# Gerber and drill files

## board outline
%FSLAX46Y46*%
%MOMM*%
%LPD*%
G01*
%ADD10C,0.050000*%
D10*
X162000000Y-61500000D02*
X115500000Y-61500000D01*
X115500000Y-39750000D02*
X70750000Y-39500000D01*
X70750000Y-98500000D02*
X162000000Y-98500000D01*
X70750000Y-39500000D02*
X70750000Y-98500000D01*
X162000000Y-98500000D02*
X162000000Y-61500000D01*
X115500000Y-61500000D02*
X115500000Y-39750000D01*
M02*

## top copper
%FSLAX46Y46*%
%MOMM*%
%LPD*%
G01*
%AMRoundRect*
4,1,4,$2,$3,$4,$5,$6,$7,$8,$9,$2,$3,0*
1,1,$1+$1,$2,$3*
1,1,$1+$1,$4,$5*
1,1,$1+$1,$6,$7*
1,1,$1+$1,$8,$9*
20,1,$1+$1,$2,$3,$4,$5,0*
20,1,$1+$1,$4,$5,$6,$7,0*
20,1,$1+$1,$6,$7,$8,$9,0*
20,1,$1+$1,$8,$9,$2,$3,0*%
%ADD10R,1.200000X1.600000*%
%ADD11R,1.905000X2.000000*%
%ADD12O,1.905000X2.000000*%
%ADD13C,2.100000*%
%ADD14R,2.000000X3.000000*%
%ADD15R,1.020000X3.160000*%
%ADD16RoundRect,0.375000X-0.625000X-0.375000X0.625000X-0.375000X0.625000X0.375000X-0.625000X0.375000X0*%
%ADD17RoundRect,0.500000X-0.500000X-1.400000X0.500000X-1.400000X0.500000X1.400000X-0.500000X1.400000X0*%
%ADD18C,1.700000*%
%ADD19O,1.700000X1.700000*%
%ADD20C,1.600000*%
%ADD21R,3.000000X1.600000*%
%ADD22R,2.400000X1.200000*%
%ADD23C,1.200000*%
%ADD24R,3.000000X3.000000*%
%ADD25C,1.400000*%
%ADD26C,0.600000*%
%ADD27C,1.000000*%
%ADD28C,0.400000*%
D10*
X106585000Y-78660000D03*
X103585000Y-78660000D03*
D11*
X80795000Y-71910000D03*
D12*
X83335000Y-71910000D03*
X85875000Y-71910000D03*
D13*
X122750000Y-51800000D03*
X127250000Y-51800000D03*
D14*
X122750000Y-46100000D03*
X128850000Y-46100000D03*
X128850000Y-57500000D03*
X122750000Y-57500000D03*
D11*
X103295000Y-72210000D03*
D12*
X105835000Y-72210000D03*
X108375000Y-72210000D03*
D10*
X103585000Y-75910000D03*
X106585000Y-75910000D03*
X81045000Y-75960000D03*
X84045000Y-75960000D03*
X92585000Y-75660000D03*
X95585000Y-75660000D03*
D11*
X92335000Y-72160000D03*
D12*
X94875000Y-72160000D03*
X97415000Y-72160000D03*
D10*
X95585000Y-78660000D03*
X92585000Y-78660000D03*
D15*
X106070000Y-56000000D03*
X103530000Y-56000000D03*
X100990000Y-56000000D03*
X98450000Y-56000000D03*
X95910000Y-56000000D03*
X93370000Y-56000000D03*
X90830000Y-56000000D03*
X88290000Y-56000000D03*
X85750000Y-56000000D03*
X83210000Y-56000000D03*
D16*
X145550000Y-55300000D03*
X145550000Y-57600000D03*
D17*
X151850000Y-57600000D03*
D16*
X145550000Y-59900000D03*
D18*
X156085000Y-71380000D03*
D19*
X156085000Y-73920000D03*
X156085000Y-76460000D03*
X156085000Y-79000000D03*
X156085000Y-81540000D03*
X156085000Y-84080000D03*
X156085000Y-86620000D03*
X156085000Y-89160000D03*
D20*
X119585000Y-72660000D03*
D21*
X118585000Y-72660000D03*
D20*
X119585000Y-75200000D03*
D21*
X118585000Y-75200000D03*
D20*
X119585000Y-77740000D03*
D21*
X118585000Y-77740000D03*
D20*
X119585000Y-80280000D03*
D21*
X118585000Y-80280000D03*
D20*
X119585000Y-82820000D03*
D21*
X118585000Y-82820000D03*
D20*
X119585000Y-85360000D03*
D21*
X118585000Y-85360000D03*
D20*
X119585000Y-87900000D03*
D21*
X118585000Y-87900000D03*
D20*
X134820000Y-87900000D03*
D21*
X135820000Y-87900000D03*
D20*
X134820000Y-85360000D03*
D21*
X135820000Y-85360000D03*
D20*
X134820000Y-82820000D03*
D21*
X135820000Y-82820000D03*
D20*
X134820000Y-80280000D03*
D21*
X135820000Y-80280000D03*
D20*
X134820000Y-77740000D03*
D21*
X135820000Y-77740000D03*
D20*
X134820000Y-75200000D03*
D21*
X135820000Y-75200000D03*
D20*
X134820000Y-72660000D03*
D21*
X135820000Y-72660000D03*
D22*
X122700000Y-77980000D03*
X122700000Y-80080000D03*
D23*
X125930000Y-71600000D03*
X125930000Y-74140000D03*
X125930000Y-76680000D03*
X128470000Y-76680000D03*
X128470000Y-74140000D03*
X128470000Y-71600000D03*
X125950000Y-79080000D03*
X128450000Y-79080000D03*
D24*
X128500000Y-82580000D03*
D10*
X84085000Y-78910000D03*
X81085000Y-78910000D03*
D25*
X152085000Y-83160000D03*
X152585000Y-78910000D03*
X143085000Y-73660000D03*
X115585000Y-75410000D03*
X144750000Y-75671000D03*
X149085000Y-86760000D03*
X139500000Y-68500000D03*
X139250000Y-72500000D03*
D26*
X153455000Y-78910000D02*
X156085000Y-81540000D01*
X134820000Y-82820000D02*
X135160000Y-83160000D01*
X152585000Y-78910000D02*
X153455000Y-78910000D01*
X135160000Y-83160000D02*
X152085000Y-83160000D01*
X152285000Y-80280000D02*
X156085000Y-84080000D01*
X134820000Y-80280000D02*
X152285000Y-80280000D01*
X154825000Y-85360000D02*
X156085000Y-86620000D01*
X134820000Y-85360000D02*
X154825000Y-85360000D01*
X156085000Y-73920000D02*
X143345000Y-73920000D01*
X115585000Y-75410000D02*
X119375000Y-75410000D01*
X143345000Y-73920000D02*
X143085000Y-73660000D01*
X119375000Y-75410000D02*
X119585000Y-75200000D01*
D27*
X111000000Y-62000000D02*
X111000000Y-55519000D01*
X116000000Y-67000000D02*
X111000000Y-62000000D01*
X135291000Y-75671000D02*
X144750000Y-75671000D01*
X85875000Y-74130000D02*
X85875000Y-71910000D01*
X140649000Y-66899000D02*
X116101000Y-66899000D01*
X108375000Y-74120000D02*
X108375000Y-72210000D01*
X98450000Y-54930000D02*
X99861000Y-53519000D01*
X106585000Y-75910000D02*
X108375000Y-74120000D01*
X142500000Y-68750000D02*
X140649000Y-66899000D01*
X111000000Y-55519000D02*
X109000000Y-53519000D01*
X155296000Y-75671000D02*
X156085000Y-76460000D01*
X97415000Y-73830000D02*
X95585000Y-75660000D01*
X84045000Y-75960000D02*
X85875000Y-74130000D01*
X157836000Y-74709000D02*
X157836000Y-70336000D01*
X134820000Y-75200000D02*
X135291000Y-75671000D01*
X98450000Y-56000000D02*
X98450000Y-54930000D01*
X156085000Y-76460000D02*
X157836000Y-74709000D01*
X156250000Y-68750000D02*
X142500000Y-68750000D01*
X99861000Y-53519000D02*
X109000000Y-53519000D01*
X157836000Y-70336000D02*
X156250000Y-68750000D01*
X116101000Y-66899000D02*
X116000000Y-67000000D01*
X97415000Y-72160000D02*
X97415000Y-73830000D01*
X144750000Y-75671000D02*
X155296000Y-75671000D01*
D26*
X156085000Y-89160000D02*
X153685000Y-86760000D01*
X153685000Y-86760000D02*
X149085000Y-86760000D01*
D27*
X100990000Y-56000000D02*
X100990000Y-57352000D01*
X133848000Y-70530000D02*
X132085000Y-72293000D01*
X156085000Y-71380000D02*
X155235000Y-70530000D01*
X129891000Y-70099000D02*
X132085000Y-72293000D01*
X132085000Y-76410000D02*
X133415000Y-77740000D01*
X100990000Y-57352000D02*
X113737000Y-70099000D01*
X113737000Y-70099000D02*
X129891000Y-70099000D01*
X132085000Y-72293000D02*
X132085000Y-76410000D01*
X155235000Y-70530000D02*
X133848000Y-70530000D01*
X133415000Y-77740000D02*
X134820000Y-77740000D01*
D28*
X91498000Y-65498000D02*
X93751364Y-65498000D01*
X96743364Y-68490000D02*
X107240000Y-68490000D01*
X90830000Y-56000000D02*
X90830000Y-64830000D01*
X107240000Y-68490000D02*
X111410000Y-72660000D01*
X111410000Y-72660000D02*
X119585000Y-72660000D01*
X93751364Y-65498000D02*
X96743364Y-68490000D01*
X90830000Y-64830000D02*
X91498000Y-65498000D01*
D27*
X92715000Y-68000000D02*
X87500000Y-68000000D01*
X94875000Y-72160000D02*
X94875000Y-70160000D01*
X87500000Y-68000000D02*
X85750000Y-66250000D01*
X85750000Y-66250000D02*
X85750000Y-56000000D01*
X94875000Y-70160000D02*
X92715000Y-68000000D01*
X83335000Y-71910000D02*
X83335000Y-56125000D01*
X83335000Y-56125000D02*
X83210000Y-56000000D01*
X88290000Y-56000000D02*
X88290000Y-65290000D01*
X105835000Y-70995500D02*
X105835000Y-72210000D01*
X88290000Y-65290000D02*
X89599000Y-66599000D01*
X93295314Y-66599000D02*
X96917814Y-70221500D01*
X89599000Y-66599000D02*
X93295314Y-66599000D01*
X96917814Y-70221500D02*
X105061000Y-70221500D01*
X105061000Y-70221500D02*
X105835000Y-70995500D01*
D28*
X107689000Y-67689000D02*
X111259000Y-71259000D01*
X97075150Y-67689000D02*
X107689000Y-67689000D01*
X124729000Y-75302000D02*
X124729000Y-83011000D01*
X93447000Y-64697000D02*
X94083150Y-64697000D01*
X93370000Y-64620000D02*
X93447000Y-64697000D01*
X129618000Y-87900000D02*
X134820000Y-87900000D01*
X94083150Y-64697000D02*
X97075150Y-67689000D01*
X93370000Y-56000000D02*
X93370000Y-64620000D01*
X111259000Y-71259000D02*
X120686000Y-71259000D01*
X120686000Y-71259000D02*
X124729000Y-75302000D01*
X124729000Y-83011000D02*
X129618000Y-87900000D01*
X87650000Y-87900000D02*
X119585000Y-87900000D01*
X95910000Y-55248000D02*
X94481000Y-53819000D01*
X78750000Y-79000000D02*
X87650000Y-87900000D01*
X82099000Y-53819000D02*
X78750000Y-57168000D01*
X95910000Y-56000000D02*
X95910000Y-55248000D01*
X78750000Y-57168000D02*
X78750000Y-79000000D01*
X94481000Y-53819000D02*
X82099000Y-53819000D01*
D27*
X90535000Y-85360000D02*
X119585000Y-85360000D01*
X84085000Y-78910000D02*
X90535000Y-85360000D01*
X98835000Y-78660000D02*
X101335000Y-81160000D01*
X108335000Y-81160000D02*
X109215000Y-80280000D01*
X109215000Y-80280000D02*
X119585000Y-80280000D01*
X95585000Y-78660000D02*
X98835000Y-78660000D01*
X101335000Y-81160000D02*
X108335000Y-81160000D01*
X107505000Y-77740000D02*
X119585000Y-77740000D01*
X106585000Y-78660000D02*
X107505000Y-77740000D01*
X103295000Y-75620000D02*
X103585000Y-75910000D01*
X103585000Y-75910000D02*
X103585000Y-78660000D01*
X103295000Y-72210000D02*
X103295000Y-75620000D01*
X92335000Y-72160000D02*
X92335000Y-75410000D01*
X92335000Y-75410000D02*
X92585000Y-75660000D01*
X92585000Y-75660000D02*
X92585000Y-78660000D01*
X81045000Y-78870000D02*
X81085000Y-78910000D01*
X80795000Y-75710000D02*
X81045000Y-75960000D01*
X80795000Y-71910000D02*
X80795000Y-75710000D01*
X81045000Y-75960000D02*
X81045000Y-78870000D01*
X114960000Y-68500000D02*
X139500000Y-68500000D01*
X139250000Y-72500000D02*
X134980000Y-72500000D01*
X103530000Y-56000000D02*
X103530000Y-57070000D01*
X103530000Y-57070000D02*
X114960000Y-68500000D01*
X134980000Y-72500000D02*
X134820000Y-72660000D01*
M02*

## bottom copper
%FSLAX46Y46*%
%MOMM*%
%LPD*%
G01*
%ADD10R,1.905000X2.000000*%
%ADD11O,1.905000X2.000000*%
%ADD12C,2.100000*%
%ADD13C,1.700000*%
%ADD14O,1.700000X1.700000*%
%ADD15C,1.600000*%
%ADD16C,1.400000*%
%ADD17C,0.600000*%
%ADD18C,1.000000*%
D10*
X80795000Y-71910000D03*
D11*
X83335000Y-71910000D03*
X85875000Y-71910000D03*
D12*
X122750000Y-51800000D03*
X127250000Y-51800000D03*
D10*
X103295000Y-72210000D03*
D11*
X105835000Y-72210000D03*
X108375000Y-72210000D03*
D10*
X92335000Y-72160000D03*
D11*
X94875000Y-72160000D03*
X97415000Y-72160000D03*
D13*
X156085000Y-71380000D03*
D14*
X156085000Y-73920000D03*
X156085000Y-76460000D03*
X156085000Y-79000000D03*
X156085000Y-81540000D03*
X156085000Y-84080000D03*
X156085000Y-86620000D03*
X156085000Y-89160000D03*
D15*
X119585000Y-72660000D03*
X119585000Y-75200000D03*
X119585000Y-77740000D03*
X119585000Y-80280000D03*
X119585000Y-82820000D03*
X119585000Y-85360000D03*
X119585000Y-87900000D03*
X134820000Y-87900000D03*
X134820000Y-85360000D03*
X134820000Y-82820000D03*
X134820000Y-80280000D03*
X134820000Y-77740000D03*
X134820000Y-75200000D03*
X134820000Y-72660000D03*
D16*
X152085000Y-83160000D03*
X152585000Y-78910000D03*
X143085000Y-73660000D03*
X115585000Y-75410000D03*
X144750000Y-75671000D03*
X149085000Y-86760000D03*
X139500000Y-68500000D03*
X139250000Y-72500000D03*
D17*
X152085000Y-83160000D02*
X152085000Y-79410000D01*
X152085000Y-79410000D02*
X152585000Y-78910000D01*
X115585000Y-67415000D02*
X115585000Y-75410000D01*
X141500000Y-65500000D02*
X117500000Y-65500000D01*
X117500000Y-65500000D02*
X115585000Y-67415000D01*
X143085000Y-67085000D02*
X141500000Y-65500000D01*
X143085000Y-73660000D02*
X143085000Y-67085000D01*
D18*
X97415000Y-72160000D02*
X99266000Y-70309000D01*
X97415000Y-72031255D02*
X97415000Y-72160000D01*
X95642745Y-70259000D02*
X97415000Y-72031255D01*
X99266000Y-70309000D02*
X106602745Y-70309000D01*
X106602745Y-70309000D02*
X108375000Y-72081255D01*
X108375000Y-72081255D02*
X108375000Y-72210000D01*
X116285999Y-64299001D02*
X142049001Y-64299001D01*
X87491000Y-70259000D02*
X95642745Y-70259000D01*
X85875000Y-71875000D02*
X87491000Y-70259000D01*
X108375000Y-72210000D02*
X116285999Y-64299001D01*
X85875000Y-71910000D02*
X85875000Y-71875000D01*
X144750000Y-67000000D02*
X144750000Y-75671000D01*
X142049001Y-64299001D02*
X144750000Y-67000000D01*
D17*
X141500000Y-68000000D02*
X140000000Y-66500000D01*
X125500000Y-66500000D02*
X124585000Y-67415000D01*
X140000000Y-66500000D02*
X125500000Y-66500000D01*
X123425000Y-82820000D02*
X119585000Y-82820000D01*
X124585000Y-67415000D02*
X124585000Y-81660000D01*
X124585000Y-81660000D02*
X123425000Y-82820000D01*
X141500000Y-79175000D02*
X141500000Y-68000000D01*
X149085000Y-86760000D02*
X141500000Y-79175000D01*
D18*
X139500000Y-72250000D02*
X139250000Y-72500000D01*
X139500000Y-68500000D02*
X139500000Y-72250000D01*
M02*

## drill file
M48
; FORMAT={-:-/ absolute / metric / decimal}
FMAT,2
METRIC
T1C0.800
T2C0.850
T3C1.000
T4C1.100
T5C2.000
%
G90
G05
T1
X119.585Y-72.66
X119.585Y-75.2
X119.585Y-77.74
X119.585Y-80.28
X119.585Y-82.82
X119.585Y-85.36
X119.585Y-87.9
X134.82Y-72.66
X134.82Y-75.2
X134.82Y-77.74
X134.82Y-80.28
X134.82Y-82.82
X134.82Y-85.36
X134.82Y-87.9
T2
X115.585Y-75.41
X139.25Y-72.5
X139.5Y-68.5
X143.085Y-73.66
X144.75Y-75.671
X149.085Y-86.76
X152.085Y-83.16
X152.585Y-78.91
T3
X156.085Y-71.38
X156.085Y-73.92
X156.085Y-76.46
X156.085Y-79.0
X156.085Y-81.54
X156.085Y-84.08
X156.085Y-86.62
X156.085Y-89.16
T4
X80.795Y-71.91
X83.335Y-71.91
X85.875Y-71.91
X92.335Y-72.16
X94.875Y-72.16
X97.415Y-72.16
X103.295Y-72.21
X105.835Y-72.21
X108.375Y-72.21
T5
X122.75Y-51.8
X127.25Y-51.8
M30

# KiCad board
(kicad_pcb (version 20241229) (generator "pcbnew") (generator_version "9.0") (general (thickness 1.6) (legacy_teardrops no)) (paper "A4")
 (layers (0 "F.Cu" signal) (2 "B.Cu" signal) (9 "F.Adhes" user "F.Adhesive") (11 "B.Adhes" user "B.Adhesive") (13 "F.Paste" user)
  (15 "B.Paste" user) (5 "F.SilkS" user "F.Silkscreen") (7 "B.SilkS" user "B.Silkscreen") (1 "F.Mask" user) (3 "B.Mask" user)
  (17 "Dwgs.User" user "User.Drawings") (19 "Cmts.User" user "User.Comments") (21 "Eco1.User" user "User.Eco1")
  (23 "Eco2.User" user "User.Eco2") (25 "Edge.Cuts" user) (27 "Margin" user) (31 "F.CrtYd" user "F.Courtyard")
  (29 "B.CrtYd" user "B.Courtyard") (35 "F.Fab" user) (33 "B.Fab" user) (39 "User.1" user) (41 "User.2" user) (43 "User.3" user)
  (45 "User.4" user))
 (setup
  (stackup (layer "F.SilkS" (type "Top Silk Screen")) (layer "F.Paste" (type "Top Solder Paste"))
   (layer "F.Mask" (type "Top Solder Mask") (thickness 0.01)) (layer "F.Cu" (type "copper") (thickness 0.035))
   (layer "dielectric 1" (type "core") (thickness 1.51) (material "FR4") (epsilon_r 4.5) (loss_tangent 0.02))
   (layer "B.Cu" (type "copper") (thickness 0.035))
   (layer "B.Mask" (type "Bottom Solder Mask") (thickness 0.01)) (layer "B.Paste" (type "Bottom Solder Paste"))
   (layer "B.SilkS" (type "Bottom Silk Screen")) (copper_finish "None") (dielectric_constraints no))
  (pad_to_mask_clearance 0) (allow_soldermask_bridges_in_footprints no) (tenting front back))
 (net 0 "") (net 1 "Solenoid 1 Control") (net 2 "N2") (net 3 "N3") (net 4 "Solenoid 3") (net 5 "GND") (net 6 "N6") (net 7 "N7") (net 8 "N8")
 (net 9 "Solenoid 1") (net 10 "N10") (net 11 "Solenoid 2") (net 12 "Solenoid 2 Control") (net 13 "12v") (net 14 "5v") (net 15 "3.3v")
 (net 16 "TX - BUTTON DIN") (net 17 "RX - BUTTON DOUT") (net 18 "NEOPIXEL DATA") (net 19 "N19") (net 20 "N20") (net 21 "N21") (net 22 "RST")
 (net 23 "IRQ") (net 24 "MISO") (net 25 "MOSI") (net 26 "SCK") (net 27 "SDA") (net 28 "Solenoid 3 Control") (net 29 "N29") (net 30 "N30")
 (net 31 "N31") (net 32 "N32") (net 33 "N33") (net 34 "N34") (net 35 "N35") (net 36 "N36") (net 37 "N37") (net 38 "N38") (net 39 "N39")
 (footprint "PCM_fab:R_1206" (layer "F.Cu") (at 105.085 78.66 180)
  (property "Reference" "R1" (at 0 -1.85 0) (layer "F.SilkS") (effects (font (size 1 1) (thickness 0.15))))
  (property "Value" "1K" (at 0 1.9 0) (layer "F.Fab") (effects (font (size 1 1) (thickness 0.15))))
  (pad "1" smd rect (at -1.5 0 180) (size 1.2 1.6) (layers "F.Cu" "F.Mask" "F.Paste") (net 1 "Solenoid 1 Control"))
  (pad "2" smd rect (at 1.5 0 180) (size 1.2 1.6) (layers "F.Cu" "F.Mask" "F.Paste") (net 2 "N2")))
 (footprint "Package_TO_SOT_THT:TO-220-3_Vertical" (layer "F.Cu") (at 80.795 71.91)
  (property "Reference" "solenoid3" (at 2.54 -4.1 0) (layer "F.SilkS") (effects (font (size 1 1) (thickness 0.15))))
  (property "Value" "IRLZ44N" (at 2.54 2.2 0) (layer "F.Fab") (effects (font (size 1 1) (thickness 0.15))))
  (pad "1" thru_hole rect (at 0 0) (size 1.905 2) (drill 1.1) (layers "*.Cu" "*.Mask") (remove_unused_layers no) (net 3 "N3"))
  (pad "2" thru_hole oval (at 2.54 0) (size 1.905 2) (drill 1.1) (layers "*.Cu" "*.Mask") (remove_unused_layers no) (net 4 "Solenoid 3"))
  (pad "3" thru_hole oval (at 5.08 0) (size 1.905 2) (drill 1.1) (layers "*.Cu" "*.Mask") (remove_unused_layers no) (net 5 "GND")))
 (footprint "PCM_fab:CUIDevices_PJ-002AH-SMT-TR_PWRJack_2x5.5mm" (layer "F.Cu") (at 125.75 51.8)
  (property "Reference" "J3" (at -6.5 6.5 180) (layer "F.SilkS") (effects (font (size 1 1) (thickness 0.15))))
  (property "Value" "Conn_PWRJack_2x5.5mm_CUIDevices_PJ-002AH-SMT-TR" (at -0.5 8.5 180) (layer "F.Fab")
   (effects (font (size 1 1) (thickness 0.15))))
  (pad "" thru_hole circle (at -3 0 90) (size 2.1 2.1) (drill 2) (layers "*.Cu" "*.Mask") (remove_unused_layers no))
  (pad "" thru_hole circle (at 1.5 0 90) (size 2.1 2.1) (drill 2) (layers "*.Cu" "*.Mask") (remove_unused_layers no))
  (pad "1" smd rect (at -3 -5.7 90) (size 3 2) (layers "F.Cu" "F.Mask" "F.Paste") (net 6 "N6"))
  (pad "1" smd rect (at 3.1 -5.7 90) (size 3 2) (layers "F.Cu" "F.Mask" "F.Paste") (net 6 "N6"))
  (pad "2" smd rect (at 3.1 5.7 90) (size 3 2) (layers "F.Cu" "F.Mask" "F.Paste") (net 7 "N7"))
  (pad "3" smd rect (at -3 5.7 90) (size 3 2) (layers "F.Cu" "F.Mask" "F.Paste") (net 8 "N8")))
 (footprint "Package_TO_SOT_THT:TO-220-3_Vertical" (layer "F.Cu") (at 103.295 72.21)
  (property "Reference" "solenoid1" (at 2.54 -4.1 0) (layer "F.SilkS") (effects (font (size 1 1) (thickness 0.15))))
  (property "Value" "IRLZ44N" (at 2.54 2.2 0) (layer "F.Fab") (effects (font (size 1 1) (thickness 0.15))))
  (pad "1" thru_hole rect (at 0 0) (size 1.905 2) (drill 1.1) (layers "*.Cu" "*.Mask") (remove_unused_layers no) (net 2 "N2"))
  (pad "2" thru_hole oval (at 2.54 0) (size 1.905 2) (drill 1.1) (layers "*.Cu" "*.Mask") (remove_unused_layers no) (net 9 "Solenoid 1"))
  (pad "3" thru_hole oval (at 5.08 0) (size 1.905 2) (drill 1.1) (layers "*.Cu" "*.Mask") (remove_unused_layers no) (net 5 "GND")))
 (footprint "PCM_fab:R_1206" (layer "F.Cu") (at 105.085 75.91)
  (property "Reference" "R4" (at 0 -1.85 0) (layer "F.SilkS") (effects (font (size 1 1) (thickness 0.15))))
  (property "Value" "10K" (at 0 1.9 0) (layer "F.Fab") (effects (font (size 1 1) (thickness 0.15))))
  (pad "1" smd rect (at -1.5 0) (size 1.2 1.6) (layers "F.Cu" "F.Mask" "F.Paste") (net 2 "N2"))
  (pad "2" smd rect (at 1.5 0) (size 1.2 1.6) (layers "F.Cu" "F.Mask" "F.Paste") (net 5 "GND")))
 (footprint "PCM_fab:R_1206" (layer "F.Cu") (at 82.545 75.96)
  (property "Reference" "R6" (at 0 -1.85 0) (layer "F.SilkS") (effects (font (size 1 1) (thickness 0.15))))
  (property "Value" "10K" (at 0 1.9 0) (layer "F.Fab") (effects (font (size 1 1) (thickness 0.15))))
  (pad "1" smd rect (at -1.5 0) (size 1.2 1.6) (layers "F.Cu" "F.Mask" "F.Paste") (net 3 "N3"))
  (pad "2" smd rect (at 1.5 0) (size 1.2 1.6) (layers "F.Cu" "F.Mask" "F.Paste") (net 5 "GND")))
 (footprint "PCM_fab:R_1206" (layer "F.Cu") (at 94.085 75.66)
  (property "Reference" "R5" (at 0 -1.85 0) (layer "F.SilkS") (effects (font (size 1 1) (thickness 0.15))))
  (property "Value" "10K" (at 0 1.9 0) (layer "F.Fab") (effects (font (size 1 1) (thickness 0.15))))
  (pad "1" smd rect (at -1.5 0) (size 1.2 1.6) (layers "F.Cu" "F.Mask" "F.Paste") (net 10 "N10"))
  (pad "2" smd rect (at 1.5 0) (size 1.2 1.6) (layers "F.Cu" "F.Mask" "F.Paste") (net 5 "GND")))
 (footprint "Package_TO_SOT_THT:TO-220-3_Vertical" (layer "F.Cu") (at 92.335 72.16)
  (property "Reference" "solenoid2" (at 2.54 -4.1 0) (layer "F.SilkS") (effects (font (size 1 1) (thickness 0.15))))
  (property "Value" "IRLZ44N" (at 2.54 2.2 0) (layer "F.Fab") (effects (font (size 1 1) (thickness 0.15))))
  (pad "1" thru_hole rect (at 0 0) (size 1.905 2) (drill 1.1) (layers "*.Cu" "*.Mask") (remove_unused_layers no) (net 10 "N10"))
  (pad "2" thru_hole oval (at 2.54 0) (size 1.905 2) (drill 1.1) (layers "*.Cu" "*.Mask") (remove_unused_layers no) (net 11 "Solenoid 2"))
  (pad "3" thru_hole oval (at 5.08 0) (size 1.905 2) (drill 1.1) (layers "*.Cu" "*.Mask") (remove_unused_layers no) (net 5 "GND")))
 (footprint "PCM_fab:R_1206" (layer "F.Cu") (at 94.085 78.66 180)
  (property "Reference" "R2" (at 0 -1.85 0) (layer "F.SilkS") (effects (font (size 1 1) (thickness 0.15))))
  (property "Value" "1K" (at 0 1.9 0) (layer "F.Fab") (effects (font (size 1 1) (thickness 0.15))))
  (pad "1" smd rect (at -1.5 0 180) (size 1.2 1.6) (layers "F.Cu" "F.Mask" "F.Paste") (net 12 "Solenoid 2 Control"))
  (pad "2" smd rect (at 1.5 0 180) (size 1.2 1.6) (layers "F.Cu" "F.Mask" "F.Paste") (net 10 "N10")))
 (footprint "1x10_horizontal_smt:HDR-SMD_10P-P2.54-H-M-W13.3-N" (layer "F.Cu") (at 94.64 56 180)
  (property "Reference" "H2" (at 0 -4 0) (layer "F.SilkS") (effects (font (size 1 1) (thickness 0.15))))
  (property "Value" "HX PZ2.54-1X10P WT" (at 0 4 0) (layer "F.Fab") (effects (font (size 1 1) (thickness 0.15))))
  (pad "1" smd rect (at -11.43 0 180) (size 1.02 3.16) (layers "F.Cu" "F.Mask" "F.Paste") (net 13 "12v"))
  (pad "2" smd rect (at -8.89 0 180) (size 1.02 3.16) (layers "F.Cu" "F.Mask" "F.Paste") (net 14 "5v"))
  (pad "3" smd rect (at -6.35 0 180) (size 1.02 3.16) (layers "F.Cu" "F.Mask" "F.Paste") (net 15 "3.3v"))
  (pad "4" smd rect (at -3.81 0 180) (size 1.02 3.16) (layers "F.Cu" "F.Mask" "F.Paste") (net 5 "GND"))
  (pad "5" smd rect (at -1.27 0 180) (size 1.02 3.16) (layers "F.Cu" "F.Mask" "F.Paste") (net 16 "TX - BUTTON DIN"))
  (pad "6" smd rect (at 1.27 0 180) (size 1.02 3.16) (layers "F.Cu" "F.Mask" "F.Paste") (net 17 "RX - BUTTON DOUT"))
  (pad "7" smd rect (at 3.81 0 180) (size 1.02 3.16) (layers "F.Cu" "F.Mask" "F.Paste") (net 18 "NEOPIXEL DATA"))
  (pad "8" smd rect (at 6.35 0 180) (size 1.02 3.16) (layers "F.Cu" "F.Mask" "F.Paste") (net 9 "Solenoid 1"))
  (pad "9" smd rect (at 8.89 0 180) (size 1.02 3.16) (layers "F.Cu" "F.Mask" "F.Paste") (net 11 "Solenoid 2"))
  (pad "10" smd rect (at 11.43 0 180) (size 1.02 3.16) (layers "F.Cu" "F.Mask" "F.Paste") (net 4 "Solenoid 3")))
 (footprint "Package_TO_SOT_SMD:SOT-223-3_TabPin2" (layer "F.Cu") (at 148.7 57.6)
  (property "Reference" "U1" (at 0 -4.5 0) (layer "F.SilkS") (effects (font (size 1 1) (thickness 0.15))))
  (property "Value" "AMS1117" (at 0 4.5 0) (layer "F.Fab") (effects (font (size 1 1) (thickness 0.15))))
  (pad "1" smd roundrect (at -3.15 -2.3) (size 2 1.5) (layers "F.Cu" "F.Mask" "F.Paste") (roundrect_rratio 0.25) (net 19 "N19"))
  (pad "2" smd roundrect (at -3.15 0) (size 2 1.5) (layers "F.Cu" "F.Mask" "F.Paste") (roundrect_rratio 0.25) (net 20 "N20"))
  (pad "2" smd roundrect (at 3.15 0) (size 2 3.8) (layers "F.Cu" "F.Mask" "F.Paste") (roundrect_rratio 0.25) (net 20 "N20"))
  (pad "3" smd roundrect (at -3.15 2.3) (size 2 1.5) (layers "F.Cu" "F.Mask" "F.Paste") (roundrect_rratio 0.25) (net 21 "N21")))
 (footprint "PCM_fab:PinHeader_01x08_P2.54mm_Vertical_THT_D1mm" (layer "F.Cu") (at 156.085 71.38)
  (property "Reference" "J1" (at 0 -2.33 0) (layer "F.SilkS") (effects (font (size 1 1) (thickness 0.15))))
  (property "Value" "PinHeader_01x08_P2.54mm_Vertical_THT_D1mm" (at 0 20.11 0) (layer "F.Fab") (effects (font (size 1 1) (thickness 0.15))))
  (pad "1" thru_hole circle (at 0 0) (size 1.7 1.7) (drill 1) (layers "*.Cu" "*.Mask") (remove_unused_layers no) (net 15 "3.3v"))
  (pad "2" thru_hole oval (at 0 2.54) (size 1.7 1.7) (drill 1) (layers "*.Cu" "*.Mask") (remove_unused_layers no) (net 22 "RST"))
  (pad "3" thru_hole oval (at 0 5.08) (size 1.7 1.7) (drill 1) (layers "*.Cu" "*.Mask") (remove_unused_layers no) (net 5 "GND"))
  (pad "4" thru_hole oval (at 0 7.62) (size 1.7 1.7) (drill 1) (layers "*.Cu" "*.Mask") (remove_unused_layers no) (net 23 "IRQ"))
  (pad "5" thru_hole oval (at 0 10.16) (size 1.7 1.7) (drill 1) (layers "*.Cu" "*.Mask") (remove_unused_layers no) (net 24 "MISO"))
  (pad "6" thru_hole oval (at 0 12.7) (size 1.7 1.7) (drill 1) (layers "*.Cu" "*.Mask") (remove_unused_layers no) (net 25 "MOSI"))
  (pad "7" thru_hole oval (at 0 15.24) (size 1.7 1.7) (drill 1) (layers "*.Cu" "*.Mask") (remove_unused_layers no) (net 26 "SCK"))
  (pad "8" thru_hole oval (at 0 17.78) (size 1.7 1.7) (drill 1) (layers "*.Cu" "*.Mask") (remove_unused_layers no) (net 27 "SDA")))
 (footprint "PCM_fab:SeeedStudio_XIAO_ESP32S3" (layer "F.Cu") (at 127.2 80.28)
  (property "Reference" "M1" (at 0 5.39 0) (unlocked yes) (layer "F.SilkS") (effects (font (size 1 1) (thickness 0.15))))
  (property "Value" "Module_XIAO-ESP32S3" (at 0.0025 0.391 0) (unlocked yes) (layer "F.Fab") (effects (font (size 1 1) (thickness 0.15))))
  (pad "1" thru_hole circle (at -7.615 -7.62) (size 1.6 1.6) (drill 0.8) (layers "*.Cu" "*.Mask") (remove_unused_layers no)
   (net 18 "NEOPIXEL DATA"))
  (pad "1" smd rect (at -7.615 -7.62) (size 3 1.6) (drill (offset -1 0)) (layers "F.Cu" "F.Mask" "F.Paste") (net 18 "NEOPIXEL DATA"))
  (pad "2" thru_hole circle (at -7.615 -5.08) (size 1.6 1.6) (drill 0.8) (layers "*.Cu" "*.Mask") (remove_unused_layers no) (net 22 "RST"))
  (pad "2" smd rect (at -7.615 -5.08) (size 3 1.6) (drill (offset -1 0)) (layers "F.Cu" "F.Mask" "F.Paste") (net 22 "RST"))
  (pad "3" thru_hole circle (at -7.615 -2.54) (size 1.6 1.6) (drill 0.8) (layers "*.Cu" "*.Mask") (remove_unused_layers no)
   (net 1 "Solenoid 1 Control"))
  (pad "3" smd rect (at -7.615 -2.54) (size 3 1.6) (drill (offset -1 0)) (layers "F.Cu" "F.Mask" "F.Paste") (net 1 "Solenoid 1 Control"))
  (pad "4" thru_hole circle (at -7.615 0) (size 1.6 1.6) (drill 0.8) (layers "*.Cu" "*.Mask") (remove_unused_layers no)
   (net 12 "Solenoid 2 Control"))
  (pad "4" smd rect (at -7.615 0) (size 3 1.6) (drill (offset -1 0)) (layers "F.Cu" "F.Mask" "F.Paste") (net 12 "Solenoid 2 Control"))
  (pad "5" thru_hole circle (at -7.615 2.54) (size 1.6 1.6) (drill 0.8) (layers "*.Cu" "*.Mask") (remove_unused_layers no) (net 27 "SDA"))
  (pad "5" smd rect (at -7.615 2.54) (size 3 1.6) (drill (offset -1 0)) (layers "F.Cu" "F.Mask" "F.Paste") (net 27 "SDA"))
  (pad "6" thru_hole circle (at -7.615 5.08) (size 1.6 1.6) (drill 0.8) (layers "*.Cu" "*.Mask") (remove_unused_layers no)
   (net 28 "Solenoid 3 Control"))
  (pad "6" smd rect (at -7.615 5.08) (size 3 1.6) (drill (offset -1 0)) (layers "F.Cu" "F.Mask" "F.Paste") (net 28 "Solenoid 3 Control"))
  (pad "7" thru_hole circle (at -7.615 7.62) (size 1.6 1.6) (drill 0.8) (layers "*.Cu" "*.Mask") (remove_unused_layers no)
   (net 16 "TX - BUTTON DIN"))
  (pad "7" smd rect (at -7.615 7.62) (size 3 1.6) (drill (offset -1 0)) (layers "F.Cu" "F.Mask" "F.Paste") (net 16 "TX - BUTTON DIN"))
  (pad "8" thru_hole circle (at 7.62 7.62) (size 1.6 1.6) (drill 0.8) (layers "*.Cu" "*.Mask") (remove_unused_layers no)
   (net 17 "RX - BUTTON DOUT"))
  (pad "8" smd rect (at 7.62 7.62) (size 3 1.6) (drill (offset 1 0)) (layers "F.Cu" "F.Mask" "F.Paste") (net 17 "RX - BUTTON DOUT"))
  (pad "9" thru_hole circle (at 7.62 5.08) (size 1.6 1.6) (drill 0.8) (layers "*.Cu" "*.Mask") (remove_unused_layers no) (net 26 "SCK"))
  (pad "9" smd rect (at 7.62 5.08) (size 3 1.6) (drill (offset 1 0)) (layers "F.Cu" "F.Mask" "F.Paste") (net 26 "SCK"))
  (pad "10" thru_hole circle (at 7.62 2.54) (size 1.6 1.6) (drill 0.8) (layers "*.Cu" "*.Mask") (remove_unused_layers no) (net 24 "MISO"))
  (pad "10" smd rect (at 7.62 2.54) (size 3 1.6) (drill (offset 1 0)) (layers "F.Cu" "F.Mask" "F.Paste") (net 24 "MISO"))
  (pad "11" thru_hole circle (at 7.62 0) (size 1.6 1.6) (drill 0.8) (layers "*.Cu" "*.Mask") (remove_unused_layers no) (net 25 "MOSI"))
  (pad "11" smd rect (at 7.62 0) (size 3 1.6) (drill (offset 1 0)) (layers "F.Cu" "F.Mask" "F.Paste") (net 25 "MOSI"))
  (pad "12" thru_hole circle (at 7.62 -2.54) (size 1.6 1.6) (drill 0.8) (layers "*.Cu" "*.Mask") (remove_unused_layers no) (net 15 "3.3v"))
  (pad "12" smd rect (at 7.62 -2.54) (size 3 1.6) (drill (offset 1 0)) (layers "F.Cu" "F.Mask" "F.Paste") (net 15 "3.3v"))
  (pad "13" thru_hole circle (at 7.62 -5.08) (size 1.6 1.6) (drill 0.8) (layers "*.Cu" "*.Mask") (remove_unused_layers no) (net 5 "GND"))
  (pad "13" smd rect (at 7.62 -5.08) (size 3 1.6) (drill (offset 1 0)) (layers "F.Cu" "F.Mask" "F.Paste") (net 5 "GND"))
  (pad "14" thru_hole circle (at 7.62 -7.62) (size 1.6 1.6) (drill 0.8) (layers "*.Cu" "*.Mask") (remove_unused_layers no) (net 14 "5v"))
  (pad "14" smd rect (at 7.62 -7.62) (size 3 1.6) (drill (offset 1 0)) (layers "F.Cu" "F.Mask" "F.Paste") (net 14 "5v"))
  (pad "15" smd rect (at -4.5 -2.3) (size 2.4 1.2) (layers "F.Cu" "F.Mask" "F.Paste") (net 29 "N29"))
  (pad "16" smd rect (at -4.5 -0.2) (size 2.4 1.2) (layers "F.Cu" "F.Mask" "F.Paste") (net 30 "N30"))
  (pad "17" smd circle (at -1.27 -8.68) (size 1.2 1.2) (layers "F.Cu" "F.Mask" "F.Paste") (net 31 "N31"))
  (pad "18" smd circle (at -1.27 -6.14) (size 1.2 1.2) (layers "F.Cu" "F.Mask" "F.Paste") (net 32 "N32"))
  (pad "19" smd circle (at -1.27 -3.6) (size 1.2 1.2) (layers "F.Cu" "F.Mask" "F.Paste") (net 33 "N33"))
  (pad "20" smd circle (at 1.27 -3.6) (size 1.2 1.2) (layers "F.Cu" "F.Mask" "F.Paste") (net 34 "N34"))
  (pad "21" smd circle (at 1.27 -6.14) (size 1.2 1.2) (layers "F.Cu" "F.Mask" "F.Paste") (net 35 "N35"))
  (pad "22" smd circle (at 1.27 -8.68) (size 1.2 1.2) (layers "F.Cu" "F.Mask" "F.Paste") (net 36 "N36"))
  (pad "23" smd circle (at -1.25 -1.2) (size 1.2 1.2) (layers "F.Cu" "F.Mask" "F.Paste") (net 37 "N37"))
  (pad "24" smd circle (at 1.25 -1.2) (size 1.2 1.2) (layers "F.Cu" "F.Mask" "F.Paste") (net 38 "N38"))
  (pad "25" smd rect (at 1.3 2.3) (size 3 3) (layers "F.Cu" "F.Mask" "F.Paste") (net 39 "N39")))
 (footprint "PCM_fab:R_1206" (layer "F.Cu") (at 82.585 78.91 180)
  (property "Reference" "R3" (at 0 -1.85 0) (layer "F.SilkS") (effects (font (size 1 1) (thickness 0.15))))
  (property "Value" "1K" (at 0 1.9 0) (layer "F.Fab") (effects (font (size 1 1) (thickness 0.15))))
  (pad "1" smd rect (at -1.5 0 180) (size 1.2 1.6) (layers "F.Cu" "F.Mask" "F.Paste") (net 28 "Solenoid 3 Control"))
  (pad "2" smd rect (at 1.5 0 180) (size 1.2 1.6) (layers "F.Cu" "F.Mask" "F.Paste") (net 3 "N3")))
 (gr_line (start 162 61.5) (end 115.5 61.5) (stroke (width 0.05) (type default)) (layer "Edge.Cuts"))
 (gr_line (start 115.5 39.75) (end 70.75 39.5) (stroke (width 0.05) (type default)) (layer "Edge.Cuts"))
 (gr_line (start 70.75 98.5) (end 162 98.5) (stroke (width 0.05) (type default)) (layer "Edge.Cuts"))
 (gr_line (start 70.75 39.5) (end 70.75 98.5) (stroke (width 0.05) (type default)) (layer "Edge.Cuts"))
 (gr_line (start 162 98.5) (end 162 61.5) (stroke (width 0.05) (type default)) (layer "Edge.Cuts"))
 (gr_line (start 115.5 61.5) (end 115.5 39.75) (stroke (width 0.05) (type default)) (layer "Edge.Cuts"))
 (segment (start 153.455 78.91) (end 156.085 81.54) (width 0.6) (layer "F.Cu") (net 24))
 (segment (start 134.82 82.82) (end 135.16 83.16) (width 0.6) (layer "F.Cu") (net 24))
 (segment (start 152.585 78.91) (end 153.455 78.91) (width 0.6) (layer "F.Cu") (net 24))
 (segment (start 135.16 83.16) (end 152.085 83.16) (width 0.6) (layer "F.Cu") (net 24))
 (via (at 152.085 83.16) (size 1.4) (drill 0.85) (layers "F.Cu" "B.Cu") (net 24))
 (via (at 152.585 78.91) (size 1.4) (drill 0.85) (layers "F.Cu" "B.Cu") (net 24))
 (segment (start 152.085 83.16) (end 152.085 79.41) (width 0.6) (layer "B.Cu") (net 24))
 (segment (start 152.085 79.41) (end 152.585 78.91) (width 0.6) (layer "B.Cu") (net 24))
 (segment (start 152.285 80.28) (end 156.085 84.08) (width 0.6) (layer "F.Cu") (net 25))
 (segment (start 134.82 80.28) (end 152.285 80.28) (width 0.6) (layer "F.Cu") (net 25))
 (segment (start 154.825 85.36) (end 156.085 86.62) (width 0.6) (layer "F.Cu") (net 26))
 (segment (start 134.82 85.36) (end 154.825 85.36) (width 0.6) (layer "F.Cu") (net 26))
 (segment (start 156.085 73.92) (end 143.345 73.92) (width 0.6) (layer "F.Cu") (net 22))
 (segment (start 115.585 75.41) (end 119.375 75.41) (width 0.6) (layer "F.Cu") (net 22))
 (segment (start 143.345 73.92) (end 143.085 73.66) (width 0.6) (layer "F.Cu") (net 22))
 (segment (start 119.375 75.41) (end 119.585 75.2) (width 0.6) (layer "F.Cu") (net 22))
 (via (at 143.085 73.66) (size 1.4) (drill 0.85) (layers "F.Cu" "B.Cu") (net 22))
 (via (at 115.585 75.41) (size 1.4) (drill 0.85) (layers "F.Cu" "B.Cu") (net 22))
 (segment (start 115.585 67.415) (end 115.585 75.41) (width 0.6) (layer "B.Cu") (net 22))
 (segment (start 141.5 65.5) (end 117.5 65.5) (width 0.6) (layer "B.Cu") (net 22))
 (segment (start 117.5 65.5) (end 115.585 67.415) (width 0.6) (layer "B.Cu") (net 22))
 (segment (start 143.085 67.085) (end 141.5 65.5) (width 0.6) (layer "B.Cu") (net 22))
 (segment (start 143.085 73.66) (end 143.085 67.085) (width 0.6) (layer "B.Cu") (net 22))
 (segment (start 111 62) (end 111 55.519) (width 1) (layer "F.Cu") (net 5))
 (segment (start 116 67) (end 111 62) (width 1) (layer "F.Cu") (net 5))
 (segment (start 135.291 75.671) (end 144.75 75.671) (width 1) (layer "F.Cu") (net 5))
 (segment (start 85.875 74.13) (end 85.875 71.91) (width 1) (layer "F.Cu") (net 5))
 (segment (start 140.649 66.899) (end 116.101 66.899) (width 1) (layer "F.Cu") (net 5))
 (segment (start 108.375 74.12) (end 108.375 72.21) (width 1) (layer "F.Cu") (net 5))
 (segment (start 98.45 54.93) (end 99.861 53.519) (width 1) (layer "F.Cu") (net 5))
 (segment (start 106.585 75.91) (end 108.375 74.12) (width 1) (layer "F.Cu") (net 5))
 (segment (start 142.5 68.75) (end 140.649 66.899) (width 1) (layer "F.Cu") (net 5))
 (segment (start 111 55.519) (end 109 53.519) (width 1) (layer "F.Cu") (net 5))
 (segment (start 155.296 75.671) (end 156.085 76.46) (width 1) (layer "F.Cu") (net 5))
 (segment (start 97.415 73.83) (end 95.585 75.66) (width 1) (layer "F.Cu") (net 5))
 (segment (start 84.045 75.96) (end 85.875 74.13) (width 1) (layer "F.Cu") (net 5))
 (segment (start 157.836 74.709) (end 157.836 70.336) (width 1) (layer "F.Cu") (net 5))
 (segment (start 134.82 75.2) (end 135.291 75.671) (width 1) (layer "F.Cu") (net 5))
 (segment (start 98.45 56) (end 98.45 54.93) (width 1) (layer "F.Cu") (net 5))
 (segment (start 156.085 76.46) (end 157.836 74.709) (width 1) (layer "F.Cu") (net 5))
 (segment (start 156.25 68.75) (end 142.5 68.75) (width 1) (layer "F.Cu") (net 5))
 (segment (start 99.861 53.519) (end 109 53.519) (width 1) (layer "F.Cu") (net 5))
 (segment (start 157.836 70.336) (end 156.25 68.75) (width 1) (layer "F.Cu") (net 5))
 (segment (start 116.101 66.899) (end 116 67) (width 1) (layer "F.Cu") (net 5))
 (segment (start 97.415 72.16) (end 97.415 73.83) (width 1) (layer "F.Cu") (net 5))
 (segment (start 144.75 75.671) (end 155.296 75.671) (width 1) (layer "F.Cu") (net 5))
 (via (at 144.75 75.671) (size 1.4) (drill 0.85) (layers "F.Cu" "B.Cu") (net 5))
 (segment (start 97.415 72.16) (end 99.266 70.309) (width 1) (layer "B.Cu") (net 5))
 (segment (start 97.415 72.031255) (end 97.415 72.16) (width 1) (layer "B.Cu") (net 5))
 (segment (start 95.642745 70.259) (end 97.415 72.031255) (width 1) (layer "B.Cu") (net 5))
 (segment (start 99.266 70.309) (end 106.602745 70.309) (width 1) (layer "B.Cu") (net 5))
 (segment (start 106.602745 70.309) (end 108.375 72.081255) (width 1) (layer "B.Cu") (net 5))
 (segment (start 108.375 72.081255) (end 108.375 72.21) (width 1) (layer "B.Cu") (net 5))
 (segment (start 116.285999 64.299001) (end 142.049001 64.299001) (width 1) (layer "B.Cu") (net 5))
 (segment (start 87.491 70.259) (end 95.642745 70.259) (width 1) (layer "B.Cu") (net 5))
 (segment (start 85.875 71.875) (end 87.491 70.259) (width 1) (layer "B.Cu") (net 5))
 (segment (start 108.375 72.21) (end 116.285999 64.299001) (width 1) (layer "B.Cu") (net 5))
 (segment (start 85.875 71.91) (end 85.875 71.875) (width 1) (layer "B.Cu") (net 5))
 (segment (start 144.75 67) (end 144.75 75.671) (width 1) (layer "B.Cu") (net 5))
 (segment (start 142.049001 64.299001) (end 144.75 67) (width 1) (layer "B.Cu") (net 5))
 (segment (start 156.085 89.16) (end 153.685 86.76) (width 0.6) (layer "F.Cu") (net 27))
 (segment (start 153.685 86.76) (end 149.085 86.76) (width 0.6) (layer "F.Cu") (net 27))
 (via (at 149.085 86.76) (size 1.4) (drill 0.85) (layers "F.Cu" "B.Cu") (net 27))
 (segment (start 141.5 68) (end 140 66.5) (width 0.6) (layer "B.Cu") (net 27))
 (segment (start 125.5 66.5) (end 124.585 67.415) (width 0.6) (layer "B.Cu") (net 27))
 (segment (start 140 66.5) (end 125.5 66.5) (width 0.6) (layer "B.Cu") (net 27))
 (segment (start 123.425 82.82) (end 119.585 82.82) (width 0.6) (layer "B.Cu") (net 27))
 (segment (start 124.585 67.415) (end 124.585 81.66) (width 0.6) (layer "B.Cu") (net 27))
 (segment (start 124.585 81.66) (end 123.425 82.82) (width 0.6) (layer "B.Cu") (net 27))
 (segment (start 141.5 79.175) (end 141.5 68) (width 0.6) (layer "B.Cu") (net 27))
 (segment (start 149.085 86.76) (end 141.5 79.175) (width 0.6) (layer "B.Cu") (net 27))
 (segment (start 100.99 56) (end 100.99 57.352) (width 1) (layer "F.Cu") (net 15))
 (segment (start 133.848 70.53) (end 132.085 72.293) (width 1) (layer "F.Cu") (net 15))
 (segment (start 156.085 71.38) (end 155.235 70.53) (width 1) (layer "F.Cu") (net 15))
 (segment (start 129.891 70.099) (end 132.085 72.293) (width 1) (layer "F.Cu") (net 15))
 (segment (start 132.085 76.41) (end 133.415 77.74) (width 1) (layer "F.Cu") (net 15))
 (segment (start 100.99 57.352) (end 113.737 70.099) (width 1) (layer "F.Cu") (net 15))
 (segment (start 113.737 70.099) (end 129.891 70.099) (width 1) (layer "F.Cu") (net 15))
 (segment (start 132.085 72.293) (end 132.085 76.41) (width 1) (layer "F.Cu") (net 15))
 (segment (start 155.235 70.53) (end 133.848 70.53) (width 1) (layer "F.Cu") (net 15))
 (segment (start 133.415 77.74) (end 134.82 77.74) (width 1) (layer "F.Cu") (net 15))
 (segment (start 91.498 65.498) (end 93.751364 65.498) (width 0.4) (layer "F.Cu") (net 18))
 (segment (start 96.743364 68.49) (end 107.24 68.49) (width 0.4) (layer "F.Cu") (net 18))
 (segment (start 90.83 56) (end 90.83 64.83) (width 0.4) (layer "F.Cu") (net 18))
 (segment (start 107.24 68.49) (end 111.41 72.66) (width 0.4) (layer "F.Cu") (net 18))
 (segment (start 111.41 72.66) (end 119.585 72.66) (width 0.4) (layer "F.Cu") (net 18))
 (segment (start 93.751364 65.498) (end 96.743364 68.49) (width 0.4) (layer "F.Cu") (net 18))
 (segment (start 90.83 64.83) (end 91.498 65.498) (width 0.4) (layer "F.Cu") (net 18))
 (segment (start 92.715 68) (end 87.5 68) (width 1) (layer "F.Cu") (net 11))
 (segment (start 94.875 72.16) (end 94.875 70.16) (width 1) (layer "F.Cu") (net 11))
 (segment (start 87.5 68) (end 85.75 66.25) (width 1) (layer "F.Cu") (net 11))
 (segment (start 85.75 66.25) (end 85.75 56) (width 1) (layer "F.Cu") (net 11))
 (segment (start 94.875 70.16) (end 92.715 68) (width 1) (layer "F.Cu") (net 11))
 (segment (start 83.335 71.91) (end 83.335 56.125) (width 1) (layer "F.Cu") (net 4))
 (segment (start 83.335 56.125) (end 83.21 56) (width 1) (layer "F.Cu") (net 4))
 (segment (start 88.29 56) (end 88.29 65.29) (width 1) (layer "F.Cu") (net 9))
 (segment (start 105.835 70.9955) (end 105.835 72.21) (width 1) (layer "F.Cu") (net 9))
 (segment (start 88.29 65.29) (end 89.599 66.599) (width 1) (layer "F.Cu") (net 9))
 (segment (start 93.295314 66.599) (end 96.917814 70.2215) (width 1) (layer "F.Cu") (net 9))
 (segment (start 89.599 66.599) (end 93.295314 66.599) (width 1) (layer "F.Cu") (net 9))
 (segment (start 96.917814 70.2215) (end 105.061 70.2215) (width 1) (layer "F.Cu") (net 9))
 (segment (start 105.061 70.2215) (end 105.835 70.9955) (width 1) (layer "F.Cu") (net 9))
 (segment (start 107.689 67.689) (end 111.259 71.259) (width 0.4) (layer "F.Cu") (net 17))
 (segment (start 97.07515 67.689) (end 107.689 67.689) (width 0.4) (layer "F.Cu") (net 17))
 (segment (start 124.729 75.302) (end 124.729 83.011) (width 0.4) (layer "F.Cu") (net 17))
 (segment (start 93.447 64.697) (end 94.08315 64.697) (width 0.4) (layer "F.Cu") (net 17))
 (segment (start 93.37 64.62) (end 93.447 64.697) (width 0.4) (layer "F.Cu") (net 17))
 (segment (start 129.618 87.9) (end 134.82 87.9) (width 0.4) (layer "F.Cu") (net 17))
 (segment (start 94.08315 64.697) (end 97.07515 67.689) (width 0.4) (layer "F.Cu") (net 17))
 (segment (start 93.37 56) (end 93.37 64.62) (width 0.4) (layer "F.Cu") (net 17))
 (segment (start 111.259 71.259) (end 120.686 71.259) (width 0.4) (layer "F.Cu") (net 17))
 (segment (start 120.686 71.259) (end 124.729 75.302) (width 0.4) (layer "F.Cu") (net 17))
 (segment (start 124.729 83.011) (end 129.618 87.9) (width 0.4) (layer "F.Cu") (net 17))
 (segment (start 87.65 87.9) (end 119.585 87.9) (width 0.4) (layer "F.Cu") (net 16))
 (segment (start 95.91 55.248) (end 94.481 53.819) (width 0.4) (layer "F.Cu") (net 16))
 (segment (start 78.75 79) (end 87.65 87.9) (width 0.4) (layer "F.Cu") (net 16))
 (segment (start 82.099 53.819) (end 78.75 57.168) (width 0.4) (layer "F.Cu") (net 16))
 (segment (start 95.91 56) (end 95.91 55.248) (width 0.4) (layer "F.Cu") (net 16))
 (segment (start 78.75 57.168) (end 78.75 79) (width 0.4) (layer "F.Cu") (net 16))
 (segment (start 94.481 53.819) (end 82.099 53.819) (width 0.4) (layer "F.Cu") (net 16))
 (segment (start 90.535 85.36) (end 119.585 85.36) (width 1) (layer "F.Cu") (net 28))
 (segment (start 84.085 78.91) (end 90.535 85.36) (width 1) (layer "F.Cu") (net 28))
 (segment (start 98.835 78.66) (end 101.335 81.16) (width 1) (layer "F.Cu") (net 12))
 (segment (start 108.335 81.16) (end 109.215 80.28) (width 1) (layer "F.Cu") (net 12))
 (segment (start 109.215 80.28) (end 119.585 80.28) (width 1) (layer "F.Cu") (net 12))
 (segment (start 95.585 78.66) (end 98.835 78.66) (width 1) (layer "F.Cu") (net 12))
 (segment (start 101.335 81.16) (end 108.335 81.16) (width 1) (layer "F.Cu") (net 12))
 (segment (start 107.505 77.74) (end 119.585 77.74) (width 1) (layer "F.Cu") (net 1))
 (segment (start 106.585 78.66) (end 107.505 77.74) (width 1) (layer "F.Cu") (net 1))
 (segment (start 103.295 75.62) (end 103.585 75.91) (width 1) (layer "F.Cu") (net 2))
 (segment (start 103.585 75.91) (end 103.585 78.66) (width 1) (layer "F.Cu") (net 2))
 (segment (start 103.295 72.21) (end 103.295 75.62) (width 1) (layer "F.Cu") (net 2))
 (segment (start 92.335 72.16) (end 92.335 75.41) (width 1) (layer "F.Cu") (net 10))
 (segment (start 92.335 75.41) (end 92.585 75.66) (width 1) (layer "F.Cu") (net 10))
 (segment (start 92.585 75.66) (end 92.585 78.66) (width 1) (layer "F.Cu") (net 10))
 (segment (start 81.045 78.87) (end 81.085 78.91) (width 1) (layer "F.Cu") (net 3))
 (segment (start 80.795 75.71) (end 81.045 75.96) (width 1) (layer "F.Cu") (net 3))
 (segment (start 80.795 71.91) (end 80.795 75.71) (width 1) (layer "F.Cu") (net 3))
 (segment (start 81.045 75.96) (end 81.045 78.87) (width 1) (layer "F.Cu") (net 3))
 (segment (start 114.96 68.5) (end 139.5 68.5) (width 1) (layer "F.Cu") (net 14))
 (segment (start 139.25 72.5) (end 134.98 72.5) (width 1) (layer "F.Cu") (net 14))
 (segment (start 103.53 56) (end 103.53 57.07) (width 1) (layer "F.Cu") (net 14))
 (segment (start 103.53 57.07) (end 114.96 68.5) (width 1) (layer "F.Cu") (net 14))
 (segment (start 134.98 72.5) (end 134.82 72.66) (width 1) (layer "F.Cu") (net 14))
 (via (at 139.5 68.5) (size 1.4) (drill 0.85) (layers "F.Cu" "B.Cu") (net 14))
 (via (at 139.25 72.5) (size 1.4) (drill 0.85) (layers "F.Cu" "B.Cu") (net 14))
 (segment (start 139.5 72.25) (end 139.25 72.5) (width 1) (layer "B.Cu") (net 14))
 (segment (start 139.5 68.5) (end 139.5 72.25) (width 1) (layer "B.Cu") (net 14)))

